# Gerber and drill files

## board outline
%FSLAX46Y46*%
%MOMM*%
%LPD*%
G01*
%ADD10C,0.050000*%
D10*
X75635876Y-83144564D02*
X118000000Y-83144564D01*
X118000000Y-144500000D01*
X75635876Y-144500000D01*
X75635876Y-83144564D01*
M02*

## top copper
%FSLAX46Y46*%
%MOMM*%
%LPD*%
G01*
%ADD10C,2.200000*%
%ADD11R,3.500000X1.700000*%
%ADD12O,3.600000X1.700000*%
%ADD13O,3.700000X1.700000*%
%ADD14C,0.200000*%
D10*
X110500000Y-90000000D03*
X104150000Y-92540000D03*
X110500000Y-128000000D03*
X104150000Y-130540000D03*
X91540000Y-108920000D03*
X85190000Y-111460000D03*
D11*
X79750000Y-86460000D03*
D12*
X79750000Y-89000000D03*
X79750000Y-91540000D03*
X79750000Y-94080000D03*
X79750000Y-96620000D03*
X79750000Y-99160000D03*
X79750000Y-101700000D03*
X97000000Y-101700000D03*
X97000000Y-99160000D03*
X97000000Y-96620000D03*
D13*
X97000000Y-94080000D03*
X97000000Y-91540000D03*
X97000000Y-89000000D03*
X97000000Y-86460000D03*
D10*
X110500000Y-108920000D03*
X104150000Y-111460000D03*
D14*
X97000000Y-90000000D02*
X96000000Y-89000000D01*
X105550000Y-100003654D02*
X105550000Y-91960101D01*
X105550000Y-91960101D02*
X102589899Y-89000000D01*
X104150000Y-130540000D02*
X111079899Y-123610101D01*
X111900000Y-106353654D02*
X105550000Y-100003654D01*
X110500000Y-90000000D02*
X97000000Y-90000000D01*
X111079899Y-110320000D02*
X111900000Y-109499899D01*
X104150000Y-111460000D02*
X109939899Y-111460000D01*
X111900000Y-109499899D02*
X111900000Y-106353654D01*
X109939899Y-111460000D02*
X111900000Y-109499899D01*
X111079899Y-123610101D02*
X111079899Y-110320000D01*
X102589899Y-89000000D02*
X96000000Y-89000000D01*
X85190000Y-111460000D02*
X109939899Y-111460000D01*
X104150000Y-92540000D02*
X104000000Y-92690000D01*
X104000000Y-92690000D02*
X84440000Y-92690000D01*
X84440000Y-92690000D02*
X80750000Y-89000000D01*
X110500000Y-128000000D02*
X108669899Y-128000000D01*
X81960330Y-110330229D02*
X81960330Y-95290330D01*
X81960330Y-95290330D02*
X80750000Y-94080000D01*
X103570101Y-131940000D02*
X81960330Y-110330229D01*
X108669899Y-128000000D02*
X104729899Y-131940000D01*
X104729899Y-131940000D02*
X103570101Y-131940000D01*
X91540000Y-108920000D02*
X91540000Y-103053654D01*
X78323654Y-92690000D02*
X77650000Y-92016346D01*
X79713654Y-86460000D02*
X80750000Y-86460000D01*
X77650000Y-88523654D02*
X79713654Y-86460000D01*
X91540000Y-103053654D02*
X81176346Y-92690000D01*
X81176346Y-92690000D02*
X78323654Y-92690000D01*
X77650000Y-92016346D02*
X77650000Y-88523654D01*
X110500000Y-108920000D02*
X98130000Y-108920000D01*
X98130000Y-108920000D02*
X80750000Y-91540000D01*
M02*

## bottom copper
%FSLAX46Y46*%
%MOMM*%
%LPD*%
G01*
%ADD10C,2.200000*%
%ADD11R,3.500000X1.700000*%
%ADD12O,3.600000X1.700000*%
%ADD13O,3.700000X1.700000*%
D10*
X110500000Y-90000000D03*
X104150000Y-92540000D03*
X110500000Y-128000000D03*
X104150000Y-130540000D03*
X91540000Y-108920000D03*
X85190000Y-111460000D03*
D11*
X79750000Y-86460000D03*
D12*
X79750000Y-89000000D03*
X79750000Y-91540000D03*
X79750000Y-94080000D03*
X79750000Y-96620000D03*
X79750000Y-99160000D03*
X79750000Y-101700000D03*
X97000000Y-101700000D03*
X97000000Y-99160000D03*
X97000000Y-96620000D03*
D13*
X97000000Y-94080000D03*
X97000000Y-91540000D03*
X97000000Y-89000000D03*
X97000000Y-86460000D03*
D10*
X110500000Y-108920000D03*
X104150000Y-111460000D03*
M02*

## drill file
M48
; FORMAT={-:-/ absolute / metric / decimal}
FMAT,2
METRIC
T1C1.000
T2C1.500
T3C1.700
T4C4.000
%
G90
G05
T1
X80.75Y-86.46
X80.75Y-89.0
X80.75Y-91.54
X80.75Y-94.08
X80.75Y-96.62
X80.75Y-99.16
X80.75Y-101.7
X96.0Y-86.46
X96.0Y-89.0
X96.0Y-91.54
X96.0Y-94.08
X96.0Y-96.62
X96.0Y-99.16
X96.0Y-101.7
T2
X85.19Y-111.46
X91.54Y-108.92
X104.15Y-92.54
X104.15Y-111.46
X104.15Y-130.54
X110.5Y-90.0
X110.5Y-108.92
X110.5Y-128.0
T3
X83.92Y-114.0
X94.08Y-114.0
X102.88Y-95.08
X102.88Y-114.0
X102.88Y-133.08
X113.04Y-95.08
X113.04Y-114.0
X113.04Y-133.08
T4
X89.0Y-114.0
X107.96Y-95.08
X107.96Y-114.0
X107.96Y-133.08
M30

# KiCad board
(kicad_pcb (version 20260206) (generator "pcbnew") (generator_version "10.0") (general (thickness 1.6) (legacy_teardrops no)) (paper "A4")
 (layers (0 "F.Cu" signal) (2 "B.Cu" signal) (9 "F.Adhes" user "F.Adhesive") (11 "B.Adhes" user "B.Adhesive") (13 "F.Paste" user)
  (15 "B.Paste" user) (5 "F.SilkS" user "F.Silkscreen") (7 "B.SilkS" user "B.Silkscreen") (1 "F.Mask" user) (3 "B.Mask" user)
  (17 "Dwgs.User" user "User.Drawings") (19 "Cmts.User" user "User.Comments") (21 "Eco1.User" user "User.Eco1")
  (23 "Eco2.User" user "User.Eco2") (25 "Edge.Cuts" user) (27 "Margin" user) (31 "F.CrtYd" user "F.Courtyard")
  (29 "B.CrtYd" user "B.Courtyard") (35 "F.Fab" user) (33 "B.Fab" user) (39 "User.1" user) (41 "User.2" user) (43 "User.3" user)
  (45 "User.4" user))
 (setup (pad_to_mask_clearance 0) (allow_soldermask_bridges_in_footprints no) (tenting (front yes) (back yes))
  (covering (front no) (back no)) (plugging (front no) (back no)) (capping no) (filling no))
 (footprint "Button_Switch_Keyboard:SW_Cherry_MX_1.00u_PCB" (layer "F.Cu") (at 110.5 90)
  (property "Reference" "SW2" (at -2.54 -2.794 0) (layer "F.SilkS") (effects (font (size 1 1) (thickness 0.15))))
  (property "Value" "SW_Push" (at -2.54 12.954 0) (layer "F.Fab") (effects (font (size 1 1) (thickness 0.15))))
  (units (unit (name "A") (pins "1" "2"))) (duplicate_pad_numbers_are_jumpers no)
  (pad "" np_thru_hole circle (at -7.62 5.08) (size 1.7 1.7) (drill 1.7) (layers "*.Cu" "*.Mask"))
  (pad "" np_thru_hole circle (at -2.54 5.08) (size 4 4) (drill 4) (layers "*.Cu" "*.Mask"))
  (pad "" np_thru_hole circle (at 2.54 5.08) (size 1.7 1.7) (drill 1.7) (layers "*.Cu" "*.Mask"))
  (pad "1" thru_hole circle (at 0 0) (size 2.2 2.2) (drill 1.5) (layers "*.Cu" "*.Mask") (remove_unused_layers no) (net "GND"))
  (pad "2" thru_hole circle (at -6.35 2.54) (size 2.2 2.2) (drill 1.5) (layers "*.Cu" "*.Mask") (remove_unused_layers no)
   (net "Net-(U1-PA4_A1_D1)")))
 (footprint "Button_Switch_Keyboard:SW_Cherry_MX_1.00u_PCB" (layer "F.Cu") (at 110.5 128)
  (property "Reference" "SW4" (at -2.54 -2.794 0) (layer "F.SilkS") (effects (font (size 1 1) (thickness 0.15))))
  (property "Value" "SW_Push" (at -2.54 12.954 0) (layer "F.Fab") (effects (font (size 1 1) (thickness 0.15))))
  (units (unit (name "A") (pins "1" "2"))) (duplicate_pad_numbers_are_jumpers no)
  (pad "" np_thru_hole circle (at -7.62 5.08) (size 1.7 1.7) (drill 1.7) (layers "*.Cu" "*.Mask"))
  (pad "" np_thru_hole circle (at -2.54 5.08) (size 4 4) (drill 4) (layers "*.Cu" "*.Mask"))
  (pad "" np_thru_hole circle (at 2.54 5.08) (size 1.7 1.7) (drill 1.7) (layers "*.Cu" "*.Mask"))
  (pad "1" thru_hole circle (at 0 0) (size 2.2 2.2) (drill 1.5) (layers "*.Cu" "*.Mask") (remove_unused_layers no)
   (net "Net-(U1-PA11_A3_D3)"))
  (pad "2" thru_hole circle (at -6.35 2.54) (size 2.2 2.2) (drill 1.5) (layers "*.Cu" "*.Mask") (remove_unused_layers no) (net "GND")))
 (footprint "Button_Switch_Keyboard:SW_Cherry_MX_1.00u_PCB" (layer "F.Cu") (at 91.54 108.92)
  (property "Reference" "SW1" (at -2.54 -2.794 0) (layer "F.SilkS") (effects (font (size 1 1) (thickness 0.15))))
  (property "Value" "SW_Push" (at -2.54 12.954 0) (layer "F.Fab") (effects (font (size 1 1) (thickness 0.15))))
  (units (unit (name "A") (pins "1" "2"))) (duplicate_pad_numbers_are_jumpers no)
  (pad "" np_thru_hole circle (at -7.62 5.08) (size 1.7 1.7) (drill 1.7) (layers "*.Cu" "*.Mask"))
  (pad "" np_thru_hole circle (at -2.54 5.08) (size 4 4) (drill 4) (layers "*.Cu" "*.Mask"))
  (pad "" np_thru_hole circle (at 2.54 5.08) (size 1.7 1.7) (drill 1.7) (layers "*.Cu" "*.Mask"))
  (pad "1" thru_hole circle (at 0 0) (size 2.2 2.2) (drill 1.5) (layers "*.Cu" "*.Mask") (remove_unused_layers no)
   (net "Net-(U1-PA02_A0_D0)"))
  (pad "2" thru_hole circle (at -6.35 2.54) (size 2.2 2.2) (drill 1.5) (layers "*.Cu" "*.Mask") (remove_unused_layers no) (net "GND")))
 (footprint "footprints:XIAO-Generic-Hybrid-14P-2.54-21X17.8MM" (layer "F.Cu") (at 88.375 94.08)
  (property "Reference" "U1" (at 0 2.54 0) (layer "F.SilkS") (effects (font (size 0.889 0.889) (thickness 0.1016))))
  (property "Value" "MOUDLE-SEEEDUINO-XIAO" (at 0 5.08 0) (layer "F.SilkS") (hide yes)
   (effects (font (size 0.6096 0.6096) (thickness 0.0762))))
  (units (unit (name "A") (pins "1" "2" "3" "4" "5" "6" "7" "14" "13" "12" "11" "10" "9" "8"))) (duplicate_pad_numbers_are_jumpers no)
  (pad "1" thru_hole rect (at -7.625 -7.62) (size 3.5 1.7) (drill 1 (offset -1 0)) (layers "*.Cu" "*.Mask") (remove_unused_layers no)
   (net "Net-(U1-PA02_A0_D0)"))
  (pad "2" thru_hole oval (at -7.625 -5.08) (size 3.6 1.7) (drill 1 (offset -1 0)) (layers "*.Cu" "*.Mask") (remove_unused_layers no)
   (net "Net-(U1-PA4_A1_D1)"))
  (pad "3" thru_hole oval (at -7.625 -2.54) (size 3.6 1.7) (drill 1 (offset -1 0)) (layers "*.Cu" "*.Mask") (remove_unused_layers no)
   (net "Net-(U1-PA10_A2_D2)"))
  (pad "4" thru_hole oval (at -7.625 0) (size 3.6 1.7) (drill 1 (offset -1 0)) (layers "*.Cu" "*.Mask") (remove_unused_layers no)
   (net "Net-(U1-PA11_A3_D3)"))
  (pad "5" thru_hole oval (at -7.625 2.54) (size 3.6 1.7) (drill 1 (offset -1 0)) (layers "*.Cu" "*.Mask") (remove_unused_layers no)
   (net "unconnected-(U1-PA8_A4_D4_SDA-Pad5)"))
  (pad "6" thru_hole oval (at -7.625 5.08 180) (size 3.6 1.7) (drill 1 (offset 1 0)) (layers "*.Cu" "*.Mask") (remove_unused_layers no)
   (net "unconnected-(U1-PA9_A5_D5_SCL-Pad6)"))
  (pad "7" thru_hole oval (at -7.625 7.62) (size 3.6 1.7) (drill 1 (offset -1 0)) (layers "*.Cu" "*.Mask") (remove_unused_layers no)
   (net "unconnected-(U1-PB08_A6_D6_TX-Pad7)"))
  (pad "8" thru_hole oval (at 7.625 7.62) (size 3.6 1.7) (drill 1 (offset 1 0)) (layers "*.Cu" "*.Mask") (remove_unused_layers no)
   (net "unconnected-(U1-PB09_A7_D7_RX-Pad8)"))
  (pad "9" thru_hole oval (at 7.625 5.08) (size 3.6 1.7) (drill 1 (offset 1 0)) (layers "*.Cu" "*.Mask") (remove_unused_layers no)
   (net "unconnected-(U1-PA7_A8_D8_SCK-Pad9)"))
  (pad "10" thru_hole oval (at 7.625 2.54) (size 3.6 1.7) (drill 1 (offset 1 0)) (layers "*.Cu" "*.Mask") (remove_unused_layers no)
   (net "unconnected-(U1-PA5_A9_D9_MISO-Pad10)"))
  (pad "11" thru_hole oval (at 7.625 0) (size 3.7 1.7) (drill 1 (offset 1 0)) (layers "*.Cu" "*.Mask") (remove_unused_layers no)
   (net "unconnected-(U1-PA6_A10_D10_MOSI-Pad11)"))
  (pad "12" thru_hole oval (at 7.625 -2.54) (size 3.7 1.7) (drill 1 (offset 1 0)) (layers "*.Cu" "*.Mask") (remove_unused_layers no)
   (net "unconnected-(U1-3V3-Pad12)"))
  (pad "13" thru_hole oval (at 7.625 -5.08) (size 3.7 1.7) (drill 1 (offset 1 0)) (layers "*.Cu" "*.Mask") (remove_unused_layers no)
   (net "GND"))
  (pad "14" thru_hole oval (at 7.625 -7.62) (size 3.7 1.7) (drill 1 (offset 1 0)) (layers "*.Cu" "*.Mask") (remove_unused_layers no)
   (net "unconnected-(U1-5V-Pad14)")))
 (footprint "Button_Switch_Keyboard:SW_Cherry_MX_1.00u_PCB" (layer "F.Cu") (at 110.5 108.92)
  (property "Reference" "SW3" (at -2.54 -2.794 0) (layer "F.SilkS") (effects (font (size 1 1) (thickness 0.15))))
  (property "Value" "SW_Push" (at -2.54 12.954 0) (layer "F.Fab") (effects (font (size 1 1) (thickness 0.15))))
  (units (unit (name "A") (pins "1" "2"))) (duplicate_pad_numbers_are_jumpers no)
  (pad "" np_thru_hole circle (at -7.62 5.08) (size 1.7 1.7) (drill 1.7) (layers "*.Cu" "*.Mask"))
  (pad "" np_thru_hole circle (at -2.54 5.08) (size 4 4) (drill 4) (layers "*.Cu" "*.Mask"))
  (pad "" np_thru_hole circle (at 2.54 5.08) (size 1.7 1.7) (drill 1.7) (layers "*.Cu" "*.Mask"))
  (pad "1" thru_hole circle (at 0 0) (size 2.2 2.2) (drill 1.5) (layers "*.Cu" "*.Mask") (remove_unused_layers no)
   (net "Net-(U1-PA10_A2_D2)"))
  (pad "2" thru_hole circle (at -6.35 2.54) (size 2.2 2.2) (drill 1.5) (layers "*.Cu" "*.Mask") (remove_unused_layers no) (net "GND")))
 (gr_rect (start 75.635876 83.144564) (end 118 144.5) (stroke (width 0.05) (type default)) (fill no) (layer "Edge.Cuts"))
 (segment (start 97 90) (end 96 89) (width 0.2) (layer "F.Cu") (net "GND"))
 (segment (start 105.55 100.003654) (end 105.55 91.960101) (width 0.2) (layer "F.Cu") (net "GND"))
 (segment (start 105.55 91.960101) (end 102.589899 89) (width 0.2) (layer "F.Cu") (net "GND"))
 (segment (start 104.15 130.54) (end 111.079899 123.610101) (width 0.2) (layer "F.Cu") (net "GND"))
 (segment (start 111.9 106.353654) (end 105.55 100.003654) (width 0.2) (layer "F.Cu") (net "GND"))
 (segment (start 110.5 90) (end 97 90) (width 0.2) (layer "F.Cu") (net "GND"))
 (segment (start 111.079899 110.32) (end 111.9 109.499899) (width 0.2) (layer "F.Cu") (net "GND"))
 (segment (start 104.15 111.46) (end 109.939899 111.46) (width 0.2) (layer "F.Cu") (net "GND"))
 (segment (start 111.9 109.499899) (end 111.9 106.353654) (width 0.2) (layer "F.Cu") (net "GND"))
 (segment (start 109.939899 111.46) (end 111.9 109.499899) (width 0.2) (layer "F.Cu") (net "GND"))
 (segment (start 111.079899 123.610101) (end 111.079899 110.32) (width 0.2) (layer "F.Cu") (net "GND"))
 (segment (start 102.589899 89) (end 96 89) (width 0.2) (layer "F.Cu") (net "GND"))
 (segment (start 85.19 111.46) (end 109.939899 111.46) (width 0.2) (layer "F.Cu") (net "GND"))
 (segment (start 104.15 92.54) (end 104 92.69) (width 0.2) (layer "F.Cu") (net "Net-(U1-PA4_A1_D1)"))
 (segment (start 104 92.69) (end 84.44 92.69) (width 0.2) (layer "F.Cu") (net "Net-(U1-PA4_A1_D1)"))
 (segment (start 84.44 92.69) (end 80.75 89) (width 0.2) (layer "F.Cu") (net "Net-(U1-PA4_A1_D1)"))
 (segment (start 110.5 128) (end 108.669899 128) (width 0.2) (layer "F.Cu") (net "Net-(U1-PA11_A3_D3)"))
 (segment (start 81.96033 110.330229) (end 81.96033 95.29033) (width 0.2) (layer "F.Cu") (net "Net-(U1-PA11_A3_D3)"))
 (segment (start 81.96033 95.29033) (end 80.75 94.08) (width 0.2) (layer "F.Cu") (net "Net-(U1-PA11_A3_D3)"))
 (segment (start 103.570101 131.94) (end 81.96033 110.330229) (width 0.2) (layer "F.Cu") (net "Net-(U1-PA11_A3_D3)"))
 (segment (start 108.669899 128) (end 104.729899 131.94) (width 0.2) (layer "F.Cu") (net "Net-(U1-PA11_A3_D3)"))
 (segment (start 104.729899 131.94) (end 103.570101 131.94) (width 0.2) (layer "F.Cu") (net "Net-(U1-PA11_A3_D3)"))
 (segment (start 91.54 108.92) (end 91.54 103.053654) (width 0.2) (layer "F.Cu") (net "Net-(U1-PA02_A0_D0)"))
 (segment (start 78.323654 92.69) (end 77.65 92.016346) (width 0.2) (layer "F.Cu") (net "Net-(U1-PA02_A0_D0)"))
 (segment (start 79.713654 86.46) (end 80.75 86.46) (width 0.2) (layer "F.Cu") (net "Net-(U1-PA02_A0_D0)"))
 (segment (start 77.65 88.523654) (end 79.713654 86.46) (width 0.2) (layer "F.Cu") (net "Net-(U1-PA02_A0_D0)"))
 (segment (start 91.54 103.053654) (end 81.176346 92.69) (width 0.2) (layer "F.Cu") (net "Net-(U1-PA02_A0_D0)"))
 (segment (start 81.176346 92.69) (end 78.323654 92.69) (width 0.2) (layer "F.Cu") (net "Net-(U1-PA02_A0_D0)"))
 (segment (start 77.65 92.016346) (end 77.65 88.523654) (width 0.2) (layer "F.Cu") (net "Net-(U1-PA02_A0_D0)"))
 (segment (start 110.5 108.92) (end 98.13 108.92) (width 0.2) (layer "F.Cu") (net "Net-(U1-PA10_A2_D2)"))
 (segment (start 98.13 108.92) (end 80.75 91.54) (width 0.2) (layer "F.Cu") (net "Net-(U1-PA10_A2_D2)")))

